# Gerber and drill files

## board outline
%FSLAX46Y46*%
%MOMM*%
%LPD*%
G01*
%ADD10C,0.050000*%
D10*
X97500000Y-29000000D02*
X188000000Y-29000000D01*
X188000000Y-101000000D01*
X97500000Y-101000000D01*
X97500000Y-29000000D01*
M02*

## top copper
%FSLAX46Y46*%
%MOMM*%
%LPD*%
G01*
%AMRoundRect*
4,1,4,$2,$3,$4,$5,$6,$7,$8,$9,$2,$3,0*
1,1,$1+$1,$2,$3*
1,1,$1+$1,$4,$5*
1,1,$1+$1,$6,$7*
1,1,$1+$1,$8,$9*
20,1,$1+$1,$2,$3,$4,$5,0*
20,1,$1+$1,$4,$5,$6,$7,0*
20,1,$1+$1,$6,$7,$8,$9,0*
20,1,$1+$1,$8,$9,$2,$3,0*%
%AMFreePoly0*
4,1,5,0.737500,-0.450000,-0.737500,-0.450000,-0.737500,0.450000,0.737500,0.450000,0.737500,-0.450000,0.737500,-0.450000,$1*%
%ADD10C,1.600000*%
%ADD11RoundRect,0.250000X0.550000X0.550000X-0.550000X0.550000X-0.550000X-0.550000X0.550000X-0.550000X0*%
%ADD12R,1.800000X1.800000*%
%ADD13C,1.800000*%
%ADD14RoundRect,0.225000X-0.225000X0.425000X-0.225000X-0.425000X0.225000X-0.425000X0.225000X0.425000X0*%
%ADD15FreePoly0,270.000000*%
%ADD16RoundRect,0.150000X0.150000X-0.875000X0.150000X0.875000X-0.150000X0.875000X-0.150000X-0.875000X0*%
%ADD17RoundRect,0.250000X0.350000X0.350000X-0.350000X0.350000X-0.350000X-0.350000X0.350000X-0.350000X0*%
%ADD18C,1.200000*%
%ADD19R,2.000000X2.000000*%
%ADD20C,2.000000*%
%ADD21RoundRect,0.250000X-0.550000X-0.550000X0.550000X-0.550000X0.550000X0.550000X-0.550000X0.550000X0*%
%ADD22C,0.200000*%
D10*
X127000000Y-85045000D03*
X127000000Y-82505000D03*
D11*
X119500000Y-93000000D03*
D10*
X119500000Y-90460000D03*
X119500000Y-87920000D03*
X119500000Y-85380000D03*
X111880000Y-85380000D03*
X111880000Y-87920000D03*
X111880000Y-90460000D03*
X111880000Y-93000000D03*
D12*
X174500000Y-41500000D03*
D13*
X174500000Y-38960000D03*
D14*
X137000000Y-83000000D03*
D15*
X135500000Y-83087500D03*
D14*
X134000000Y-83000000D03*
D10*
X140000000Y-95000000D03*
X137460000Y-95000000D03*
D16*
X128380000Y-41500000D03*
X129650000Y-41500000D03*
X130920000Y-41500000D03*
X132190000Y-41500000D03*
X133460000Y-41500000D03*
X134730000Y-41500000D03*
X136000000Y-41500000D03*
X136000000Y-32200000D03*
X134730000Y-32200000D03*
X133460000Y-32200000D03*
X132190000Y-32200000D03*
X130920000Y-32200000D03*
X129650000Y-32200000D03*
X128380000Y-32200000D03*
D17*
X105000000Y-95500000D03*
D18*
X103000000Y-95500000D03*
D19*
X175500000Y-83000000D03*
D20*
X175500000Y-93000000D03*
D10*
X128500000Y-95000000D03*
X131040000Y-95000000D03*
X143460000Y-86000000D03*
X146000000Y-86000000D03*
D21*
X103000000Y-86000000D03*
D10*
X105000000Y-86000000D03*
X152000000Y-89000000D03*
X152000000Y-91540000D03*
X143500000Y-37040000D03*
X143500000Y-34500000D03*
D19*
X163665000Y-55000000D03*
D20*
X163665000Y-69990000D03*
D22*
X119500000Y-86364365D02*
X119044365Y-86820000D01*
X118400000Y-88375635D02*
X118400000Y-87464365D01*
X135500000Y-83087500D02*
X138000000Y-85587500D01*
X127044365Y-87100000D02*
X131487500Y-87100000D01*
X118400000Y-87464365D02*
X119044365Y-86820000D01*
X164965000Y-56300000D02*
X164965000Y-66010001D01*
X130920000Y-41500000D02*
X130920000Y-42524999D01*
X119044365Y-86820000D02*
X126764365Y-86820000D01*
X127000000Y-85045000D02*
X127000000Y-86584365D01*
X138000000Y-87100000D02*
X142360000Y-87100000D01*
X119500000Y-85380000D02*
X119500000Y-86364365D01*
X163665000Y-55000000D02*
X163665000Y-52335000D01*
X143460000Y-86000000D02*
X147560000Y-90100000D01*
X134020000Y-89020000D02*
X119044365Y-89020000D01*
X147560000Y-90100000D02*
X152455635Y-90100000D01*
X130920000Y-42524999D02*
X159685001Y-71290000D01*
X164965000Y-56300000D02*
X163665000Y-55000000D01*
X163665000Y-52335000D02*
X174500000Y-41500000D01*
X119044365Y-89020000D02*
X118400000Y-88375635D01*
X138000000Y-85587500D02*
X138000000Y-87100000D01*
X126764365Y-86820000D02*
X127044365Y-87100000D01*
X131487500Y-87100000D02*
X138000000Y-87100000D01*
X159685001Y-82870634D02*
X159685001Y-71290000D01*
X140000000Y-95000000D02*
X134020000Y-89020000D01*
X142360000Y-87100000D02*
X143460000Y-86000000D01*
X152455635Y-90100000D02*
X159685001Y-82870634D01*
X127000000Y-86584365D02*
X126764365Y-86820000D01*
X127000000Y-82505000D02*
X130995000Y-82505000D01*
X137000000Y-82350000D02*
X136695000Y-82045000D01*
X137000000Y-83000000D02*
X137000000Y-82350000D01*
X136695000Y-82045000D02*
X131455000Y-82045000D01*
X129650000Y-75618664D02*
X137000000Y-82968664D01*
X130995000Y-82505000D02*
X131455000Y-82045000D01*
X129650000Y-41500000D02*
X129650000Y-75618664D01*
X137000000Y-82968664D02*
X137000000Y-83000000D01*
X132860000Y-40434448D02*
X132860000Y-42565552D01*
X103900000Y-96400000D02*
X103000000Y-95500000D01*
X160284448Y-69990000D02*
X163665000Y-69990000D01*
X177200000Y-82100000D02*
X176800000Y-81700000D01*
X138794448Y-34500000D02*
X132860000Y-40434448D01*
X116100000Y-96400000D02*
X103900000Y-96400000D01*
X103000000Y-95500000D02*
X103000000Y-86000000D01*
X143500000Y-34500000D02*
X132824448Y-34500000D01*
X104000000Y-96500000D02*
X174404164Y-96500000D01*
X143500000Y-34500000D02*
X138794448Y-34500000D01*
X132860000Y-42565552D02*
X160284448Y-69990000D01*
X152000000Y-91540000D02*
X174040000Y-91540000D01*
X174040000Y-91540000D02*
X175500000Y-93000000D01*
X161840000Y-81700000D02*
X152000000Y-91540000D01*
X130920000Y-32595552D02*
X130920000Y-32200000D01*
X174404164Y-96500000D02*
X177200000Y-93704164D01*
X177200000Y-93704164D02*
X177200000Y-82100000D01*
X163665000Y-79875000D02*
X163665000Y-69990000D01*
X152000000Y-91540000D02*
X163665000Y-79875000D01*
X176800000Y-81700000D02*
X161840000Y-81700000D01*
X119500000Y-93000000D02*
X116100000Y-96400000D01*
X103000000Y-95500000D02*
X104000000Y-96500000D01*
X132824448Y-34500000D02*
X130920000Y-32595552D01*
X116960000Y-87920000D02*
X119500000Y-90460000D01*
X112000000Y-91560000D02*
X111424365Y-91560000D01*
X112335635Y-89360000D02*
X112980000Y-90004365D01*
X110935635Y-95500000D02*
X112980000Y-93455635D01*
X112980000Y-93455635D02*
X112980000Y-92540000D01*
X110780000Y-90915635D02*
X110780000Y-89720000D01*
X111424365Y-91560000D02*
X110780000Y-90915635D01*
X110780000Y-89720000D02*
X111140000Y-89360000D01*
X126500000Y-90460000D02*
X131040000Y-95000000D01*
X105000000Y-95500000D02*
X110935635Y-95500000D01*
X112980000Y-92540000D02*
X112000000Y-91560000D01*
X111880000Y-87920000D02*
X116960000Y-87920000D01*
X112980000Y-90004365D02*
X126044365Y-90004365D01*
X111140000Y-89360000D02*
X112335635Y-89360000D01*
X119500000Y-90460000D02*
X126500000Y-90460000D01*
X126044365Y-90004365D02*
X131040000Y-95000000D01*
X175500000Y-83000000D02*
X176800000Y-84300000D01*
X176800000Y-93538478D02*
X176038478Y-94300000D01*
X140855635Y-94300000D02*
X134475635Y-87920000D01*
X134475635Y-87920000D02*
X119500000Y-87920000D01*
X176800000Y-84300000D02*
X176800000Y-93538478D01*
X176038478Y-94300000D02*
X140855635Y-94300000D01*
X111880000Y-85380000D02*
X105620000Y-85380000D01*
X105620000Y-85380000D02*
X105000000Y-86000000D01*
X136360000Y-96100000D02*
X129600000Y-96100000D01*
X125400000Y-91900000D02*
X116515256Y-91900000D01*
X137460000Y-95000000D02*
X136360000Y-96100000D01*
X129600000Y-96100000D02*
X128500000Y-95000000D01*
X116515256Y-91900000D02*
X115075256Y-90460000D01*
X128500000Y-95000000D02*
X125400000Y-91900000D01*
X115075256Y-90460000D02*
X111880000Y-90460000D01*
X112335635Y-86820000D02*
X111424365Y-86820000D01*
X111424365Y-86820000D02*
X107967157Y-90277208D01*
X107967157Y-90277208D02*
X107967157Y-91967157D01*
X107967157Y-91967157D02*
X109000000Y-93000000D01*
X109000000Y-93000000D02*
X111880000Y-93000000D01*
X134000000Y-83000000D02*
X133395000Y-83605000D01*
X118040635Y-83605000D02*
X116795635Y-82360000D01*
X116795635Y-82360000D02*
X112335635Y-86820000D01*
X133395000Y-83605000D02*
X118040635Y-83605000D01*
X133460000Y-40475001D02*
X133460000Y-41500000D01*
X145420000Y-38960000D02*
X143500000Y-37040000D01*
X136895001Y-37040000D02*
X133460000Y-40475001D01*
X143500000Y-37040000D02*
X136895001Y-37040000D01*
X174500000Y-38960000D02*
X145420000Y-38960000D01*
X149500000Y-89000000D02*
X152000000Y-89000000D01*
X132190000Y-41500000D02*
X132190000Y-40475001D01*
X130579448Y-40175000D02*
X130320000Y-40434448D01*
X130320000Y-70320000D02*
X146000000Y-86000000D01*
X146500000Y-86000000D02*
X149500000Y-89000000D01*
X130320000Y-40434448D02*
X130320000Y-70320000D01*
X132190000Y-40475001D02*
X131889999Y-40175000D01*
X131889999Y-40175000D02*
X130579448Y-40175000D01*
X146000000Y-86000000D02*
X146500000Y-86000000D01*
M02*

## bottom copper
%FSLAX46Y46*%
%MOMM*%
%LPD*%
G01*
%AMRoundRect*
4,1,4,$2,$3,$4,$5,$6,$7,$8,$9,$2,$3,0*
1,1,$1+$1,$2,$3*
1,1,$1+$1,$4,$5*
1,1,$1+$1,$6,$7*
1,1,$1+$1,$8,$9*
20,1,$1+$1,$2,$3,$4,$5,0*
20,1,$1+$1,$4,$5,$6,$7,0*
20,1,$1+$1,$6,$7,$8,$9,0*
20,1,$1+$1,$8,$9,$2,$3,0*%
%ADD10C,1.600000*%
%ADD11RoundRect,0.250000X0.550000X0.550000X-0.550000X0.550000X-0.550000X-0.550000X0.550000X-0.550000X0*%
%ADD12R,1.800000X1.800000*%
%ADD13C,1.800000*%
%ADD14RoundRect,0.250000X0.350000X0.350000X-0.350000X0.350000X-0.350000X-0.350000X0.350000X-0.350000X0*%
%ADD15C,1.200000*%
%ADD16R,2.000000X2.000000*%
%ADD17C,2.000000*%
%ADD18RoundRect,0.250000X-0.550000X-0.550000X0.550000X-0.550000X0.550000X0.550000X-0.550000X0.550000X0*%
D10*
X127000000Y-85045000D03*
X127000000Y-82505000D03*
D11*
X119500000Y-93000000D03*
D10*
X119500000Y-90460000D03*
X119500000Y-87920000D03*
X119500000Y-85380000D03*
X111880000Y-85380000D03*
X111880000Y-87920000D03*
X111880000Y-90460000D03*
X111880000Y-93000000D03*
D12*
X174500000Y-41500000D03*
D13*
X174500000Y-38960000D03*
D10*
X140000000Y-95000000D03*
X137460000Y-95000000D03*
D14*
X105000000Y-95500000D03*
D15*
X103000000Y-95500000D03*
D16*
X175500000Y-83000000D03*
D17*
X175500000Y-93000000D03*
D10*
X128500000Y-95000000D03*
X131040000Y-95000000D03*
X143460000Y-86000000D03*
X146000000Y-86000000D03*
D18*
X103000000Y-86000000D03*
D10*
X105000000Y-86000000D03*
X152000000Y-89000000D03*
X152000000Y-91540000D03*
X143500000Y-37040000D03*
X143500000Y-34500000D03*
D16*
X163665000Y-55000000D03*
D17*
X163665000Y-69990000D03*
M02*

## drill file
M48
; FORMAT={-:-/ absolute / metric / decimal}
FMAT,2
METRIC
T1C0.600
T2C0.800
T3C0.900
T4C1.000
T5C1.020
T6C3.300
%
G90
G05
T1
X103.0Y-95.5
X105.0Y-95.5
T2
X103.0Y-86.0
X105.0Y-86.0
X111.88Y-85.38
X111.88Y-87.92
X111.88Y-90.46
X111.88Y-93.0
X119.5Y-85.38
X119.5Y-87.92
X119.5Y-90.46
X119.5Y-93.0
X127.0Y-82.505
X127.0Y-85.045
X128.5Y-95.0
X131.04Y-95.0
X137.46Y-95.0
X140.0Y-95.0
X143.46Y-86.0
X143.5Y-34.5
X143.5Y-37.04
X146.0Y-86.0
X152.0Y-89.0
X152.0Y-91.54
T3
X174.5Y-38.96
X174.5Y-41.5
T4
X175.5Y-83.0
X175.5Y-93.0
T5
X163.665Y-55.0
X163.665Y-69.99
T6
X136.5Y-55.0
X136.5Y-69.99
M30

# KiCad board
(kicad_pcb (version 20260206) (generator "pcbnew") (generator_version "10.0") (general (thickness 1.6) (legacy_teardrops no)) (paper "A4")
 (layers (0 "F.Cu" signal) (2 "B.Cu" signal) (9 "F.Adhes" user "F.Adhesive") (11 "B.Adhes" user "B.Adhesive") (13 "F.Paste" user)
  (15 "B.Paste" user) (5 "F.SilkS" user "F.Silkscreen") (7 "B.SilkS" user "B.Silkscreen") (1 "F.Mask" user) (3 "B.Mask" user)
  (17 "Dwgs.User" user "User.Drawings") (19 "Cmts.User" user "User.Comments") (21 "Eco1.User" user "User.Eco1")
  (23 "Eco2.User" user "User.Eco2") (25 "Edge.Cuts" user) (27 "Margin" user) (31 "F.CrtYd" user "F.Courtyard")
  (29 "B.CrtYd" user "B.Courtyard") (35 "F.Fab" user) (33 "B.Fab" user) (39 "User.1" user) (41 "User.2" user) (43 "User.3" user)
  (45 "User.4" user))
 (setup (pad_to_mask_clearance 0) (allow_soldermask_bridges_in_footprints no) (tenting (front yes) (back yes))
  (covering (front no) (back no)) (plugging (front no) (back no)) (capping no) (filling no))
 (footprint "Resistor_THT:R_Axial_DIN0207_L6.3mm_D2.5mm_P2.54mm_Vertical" (layer "F.Cu") (at 127 85.045 90)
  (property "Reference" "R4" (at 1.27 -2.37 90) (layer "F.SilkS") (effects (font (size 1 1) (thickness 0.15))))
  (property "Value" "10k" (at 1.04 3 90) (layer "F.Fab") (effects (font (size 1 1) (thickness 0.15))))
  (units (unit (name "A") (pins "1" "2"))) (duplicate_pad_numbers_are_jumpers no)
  (pad "1" thru_hole circle (at 0 0 90) (size 1.6 1.6) (drill 0.8) (layers "*.Cu" "*.Mask") (remove_unused_layers no) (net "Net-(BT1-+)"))
  (pad "2" thru_hole circle (at 2.54 0 90) (size 1.6 1.6) (drill 0.8) (layers "*.Cu" "*.Mask") (remove_unused_layers no) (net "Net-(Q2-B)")))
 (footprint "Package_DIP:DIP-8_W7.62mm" (layer "F.Cu") (at 119.5 93 180)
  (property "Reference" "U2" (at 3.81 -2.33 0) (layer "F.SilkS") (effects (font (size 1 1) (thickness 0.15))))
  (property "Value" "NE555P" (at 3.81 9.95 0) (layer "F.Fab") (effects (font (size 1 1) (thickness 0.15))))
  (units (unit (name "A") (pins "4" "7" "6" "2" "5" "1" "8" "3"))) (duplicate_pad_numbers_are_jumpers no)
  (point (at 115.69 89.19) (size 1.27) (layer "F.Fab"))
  (pad "1" thru_hole roundrect (at 0 0 180) (size 1.6 1.6) (drill 0.8) (layers "*.Cu" "*.Mask") (remove_unused_layers no)
   (roundrect_rratio 0.15625) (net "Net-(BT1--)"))
  (pad "2" thru_hole circle (at 0 2.54 180) (size 1.6 1.6) (drill 0.8) (layers "*.Cu" "*.Mask") (remove_unused_layers no)
   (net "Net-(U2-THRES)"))
  (pad "3" thru_hole circle (at 0 5.08 180) (size 1.6 1.6) (drill 0.8) (layers "*.Cu" "*.Mask") (remove_unused_layers no)
   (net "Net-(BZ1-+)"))
  (pad "4" thru_hole circle (at 0 7.62 180) (size 1.6 1.6) (drill 0.8) (layers "*.Cu" "*.Mask") (remove_unused_layers no)
   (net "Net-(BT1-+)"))
  (pad "5" thru_hole circle (at 7.62 7.62 180) (size 1.6 1.6) (drill 0.8) (layers "*.Cu" "*.Mask") (remove_unused_layers no)
   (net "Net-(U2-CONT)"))
  (pad "6" thru_hole circle (at 7.62 5.08 180) (size 1.6 1.6) (drill 0.8) (layers "*.Cu" "*.Mask") (remove_unused_layers no)
   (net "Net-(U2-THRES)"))
  (pad "7" thru_hole circle (at 7.62 2.54 180) (size 1.6 1.6) (drill 0.8) (layers "*.Cu" "*.Mask") (remove_unused_layers no)
   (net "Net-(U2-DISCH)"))
  (pad "8" thru_hole circle (at 7.62 0 180) (size 1.6 1.6) (drill 0.8) (layers "*.Cu" "*.Mask") (remove_unused_layers no) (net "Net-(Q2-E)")))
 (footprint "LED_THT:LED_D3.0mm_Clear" (layer "F.Cu") (at 174.5 41.5 90)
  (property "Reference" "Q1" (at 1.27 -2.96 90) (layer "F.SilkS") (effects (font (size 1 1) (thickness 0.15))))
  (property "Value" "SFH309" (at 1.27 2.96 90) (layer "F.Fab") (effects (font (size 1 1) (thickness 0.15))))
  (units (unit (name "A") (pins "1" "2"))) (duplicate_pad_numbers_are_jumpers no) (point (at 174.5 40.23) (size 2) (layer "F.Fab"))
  (pad "1" thru_hole rect (at 0 0 90) (size 1.8 1.8) (drill 0.9) (layers "*.Cu" "*.Mask") (remove_unused_layers no) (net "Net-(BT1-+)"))
  (pad "2" thru_hole circle (at 2.54 0 90) (size 1.8 1.8) (drill 0.9) (layers "*.Cu" "*.Mask") (remove_unused_layers no) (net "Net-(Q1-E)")))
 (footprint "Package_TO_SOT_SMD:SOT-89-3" (layer "F.Cu") (at 135.5 84.95 -90)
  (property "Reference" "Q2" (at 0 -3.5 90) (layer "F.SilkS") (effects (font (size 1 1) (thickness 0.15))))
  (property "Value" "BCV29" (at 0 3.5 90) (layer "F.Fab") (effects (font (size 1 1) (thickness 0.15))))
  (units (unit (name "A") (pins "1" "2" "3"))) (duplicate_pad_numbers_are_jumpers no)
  (pad "1" smd roundrect (at -1.95 -1.5 270) (size 1.3 0.9) (layers "F.Cu" "F.Mask" "F.Paste") (roundrect_rratio 0.25) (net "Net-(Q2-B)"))
  (pad "2" smd custom (at -1.8625 0 270) (size 1.475 0.9) (layers "F.Cu" "F.Mask" "F.Paste") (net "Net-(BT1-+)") (zone_connect 2)
   (thermal_bridge_angle 45) (options (clearance outline) (anchor rect)) (primitives))
  (pad "3" smd roundrect (at -1.95 1.5 270) (size 1.3 0.9) (layers "F.Cu" "F.Mask" "F.Paste") (roundrect_rratio 0.25) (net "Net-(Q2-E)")))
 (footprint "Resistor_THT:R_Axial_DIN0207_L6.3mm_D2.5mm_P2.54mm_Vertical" (layer "F.Cu") (at 140 95 180)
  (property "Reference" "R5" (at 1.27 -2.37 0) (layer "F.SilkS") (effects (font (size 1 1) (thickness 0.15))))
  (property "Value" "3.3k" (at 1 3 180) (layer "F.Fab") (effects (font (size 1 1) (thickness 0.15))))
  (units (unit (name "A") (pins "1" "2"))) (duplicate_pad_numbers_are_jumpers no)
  (pad "1" thru_hole circle (at 0 0 180) (size 1.6 1.6) (drill 0.8) (layers "*.Cu" "*.Mask") (remove_unused_layers no) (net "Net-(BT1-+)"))
  (pad "2" thru_hole circle (at 2.54 0 180) (size 1.6 1.6) (drill 0.8) (layers "*.Cu" "*.Mask") (remove_unused_layers no)
   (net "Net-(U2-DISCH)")))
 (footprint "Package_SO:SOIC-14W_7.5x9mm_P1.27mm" (layer "F.Cu") (at 132.19 36.85 90)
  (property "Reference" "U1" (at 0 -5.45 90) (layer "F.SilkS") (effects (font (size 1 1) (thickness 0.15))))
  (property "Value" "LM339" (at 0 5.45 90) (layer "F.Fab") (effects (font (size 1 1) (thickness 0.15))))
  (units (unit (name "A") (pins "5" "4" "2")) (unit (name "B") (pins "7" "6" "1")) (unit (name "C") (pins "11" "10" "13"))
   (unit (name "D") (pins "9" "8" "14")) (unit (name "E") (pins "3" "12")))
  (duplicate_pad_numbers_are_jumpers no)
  (pad "1" smd roundrect (at -4.65 -3.81 90) (size 2.05 0.6) (layers "F.Cu" "F.Mask" "F.Paste") (roundrect_rratio 0.25))
  (pad "2" smd roundrect (at -4.65 -2.54 90) (size 2.05 0.6) (layers "F.Cu" "F.Mask" "F.Paste") (roundrect_rratio 0.25) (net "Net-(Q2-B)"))
  (pad "3" smd roundrect (at -4.65 -1.27 90) (size 2.05 0.6) (layers "F.Cu" "F.Mask" "F.Paste") (roundrect_rratio 0.25) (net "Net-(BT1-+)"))
  (pad "4" smd roundrect (at -4.65 0 90) (size 2.05 0.6) (layers "F.Cu" "F.Mask" "F.Paste") (roundrect_rratio 0.25) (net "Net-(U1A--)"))
  (pad "5" smd roundrect (at -4.65 1.27 90) (size 2.05 0.6) (layers "F.Cu" "F.Mask" "F.Paste") (roundrect_rratio 0.25) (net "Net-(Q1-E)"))
  (pad "6" smd roundrect (at -4.65 2.54 90) (size 2.05 0.6) (layers "F.Cu" "F.Mask" "F.Paste") (roundrect_rratio 0.25))
  (pad "7" smd roundrect (at -4.65 3.81 90) (size 2.05 0.6) (layers "F.Cu" "F.Mask" "F.Paste") (roundrect_rratio 0.25))
  (pad "8" smd roundrect (at 4.65 3.81 90) (size 2.05 0.6) (layers "F.Cu" "F.Mask" "F.Paste") (roundrect_rratio 0.25))
  (pad "9" smd roundrect (at 4.65 2.54 90) (size 2.05 0.6) (layers "F.Cu" "F.Mask" "F.Paste") (roundrect_rratio 0.25))
  (pad "10" smd roundrect (at 4.65 1.27 90) (size 2.05 0.6) (layers "F.Cu" "F.Mask" "F.Paste") (roundrect_rratio 0.25))
  (pad "11" smd roundrect (at 4.65 0 90) (size 2.05 0.6) (layers "F.Cu" "F.Mask" "F.Paste") (roundrect_rratio 0.25))
  (pad "12" smd roundrect (at 4.65 -1.27 90) (size 2.05 0.6) (layers "F.Cu" "F.Mask" "F.Paste") (roundrect_rratio 0.25) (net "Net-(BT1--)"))
  (pad "13" smd roundrect (at 4.65 -2.54 90) (size 2.05 0.6) (layers "F.Cu" "F.Mask" "F.Paste") (roundrect_rratio 0.25))
  (pad "14" smd roundrect (at 4.65 -3.81 90) (size 2.05 0.6) (layers "F.Cu" "F.Mask" "F.Paste") (roundrect_rratio 0.25)))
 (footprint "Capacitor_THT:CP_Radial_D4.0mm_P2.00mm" (layer "F.Cu") (at 105 95.5 180)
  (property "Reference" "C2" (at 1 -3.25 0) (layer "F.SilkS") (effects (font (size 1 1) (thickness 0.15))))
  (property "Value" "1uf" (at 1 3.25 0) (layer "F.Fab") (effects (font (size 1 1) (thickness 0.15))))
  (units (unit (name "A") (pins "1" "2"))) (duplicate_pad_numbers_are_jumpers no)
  (pad "1" thru_hole roundrect (at 0 0 180) (size 1.2 1.2) (drill 0.6) (layers "*.Cu" "*.Mask") (remove_unused_layers no)
   (roundrect_rratio 0.208333) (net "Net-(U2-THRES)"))
  (pad "2" thru_hole circle (at 2 0 180) (size 1.2 1.2) (drill 0.6) (layers "*.Cu" "*.Mask") (remove_unused_layers no) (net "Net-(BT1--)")))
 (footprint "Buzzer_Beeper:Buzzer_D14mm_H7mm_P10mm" (layer "F.Cu") (at 175.5 83 -90)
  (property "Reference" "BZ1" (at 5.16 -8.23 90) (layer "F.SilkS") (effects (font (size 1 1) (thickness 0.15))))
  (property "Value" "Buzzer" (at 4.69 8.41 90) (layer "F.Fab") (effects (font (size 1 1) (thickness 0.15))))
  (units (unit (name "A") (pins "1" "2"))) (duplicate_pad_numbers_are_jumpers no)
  (pad "1" thru_hole rect (at 0 0 270) (size 2 2) (drill 1) (layers "*.Cu" "*.Mask") (remove_unused_layers no) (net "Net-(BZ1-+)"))
  (pad "2" thru_hole circle (at 10 0 270) (size 2 2) (drill 1) (layers "*.Cu" "*.Mask") (remove_unused_layers no) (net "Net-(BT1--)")))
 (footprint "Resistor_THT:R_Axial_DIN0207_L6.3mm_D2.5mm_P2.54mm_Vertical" (layer "F.Cu") (at 128.5 95)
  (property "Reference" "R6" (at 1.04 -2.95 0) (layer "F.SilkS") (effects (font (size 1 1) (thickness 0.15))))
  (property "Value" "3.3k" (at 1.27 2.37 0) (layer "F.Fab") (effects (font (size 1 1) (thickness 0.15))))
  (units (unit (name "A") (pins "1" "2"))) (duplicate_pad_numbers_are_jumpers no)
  (pad "1" thru_hole circle (at 0 0) (size 1.6 1.6) (drill 0.8) (layers "*.Cu" "*.Mask") (remove_unused_layers no) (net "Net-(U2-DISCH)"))
  (pad "2" thru_hole circle (at 2.54 0) (size 1.6 1.6) (drill 0.8) (layers "*.Cu" "*.Mask") (remove_unused_layers no) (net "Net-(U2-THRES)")))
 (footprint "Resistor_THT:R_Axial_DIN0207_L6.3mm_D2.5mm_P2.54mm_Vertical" (layer "F.Cu") (at 143.46 86)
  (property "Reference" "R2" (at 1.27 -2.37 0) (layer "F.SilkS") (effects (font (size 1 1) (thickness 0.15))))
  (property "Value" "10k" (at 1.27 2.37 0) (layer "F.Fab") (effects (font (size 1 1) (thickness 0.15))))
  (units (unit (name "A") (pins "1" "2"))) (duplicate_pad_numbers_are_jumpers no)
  (pad "1" thru_hole circle (at 0 0) (size 1.6 1.6) (drill 0.8) (layers "*.Cu" "*.Mask") (remove_unused_layers no) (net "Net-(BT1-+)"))
  (pad "2" thru_hole circle (at 2.54 0) (size 1.6 1.6) (drill 0.8) (layers "*.Cu" "*.Mask") (remove_unused_layers no) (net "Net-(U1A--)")))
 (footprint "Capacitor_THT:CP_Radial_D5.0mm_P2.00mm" (layer "F.Cu") (at 103 86)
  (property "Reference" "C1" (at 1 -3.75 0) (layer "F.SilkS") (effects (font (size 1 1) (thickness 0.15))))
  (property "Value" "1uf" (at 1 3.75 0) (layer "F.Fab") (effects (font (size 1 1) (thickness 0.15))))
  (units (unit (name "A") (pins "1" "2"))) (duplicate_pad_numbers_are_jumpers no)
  (pad "1" thru_hole roundrect (at 0 0) (size 1.6 1.6) (drill 0.8) (layers "*.Cu" "*.Mask") (remove_unused_layers no)
   (roundrect_rratio 0.15625) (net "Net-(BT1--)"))
  (pad "2" thru_hole circle (at 2 0) (size 1.6 1.6) (drill 0.8) (layers "*.Cu" "*.Mask") (remove_unused_layers no) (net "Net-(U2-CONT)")))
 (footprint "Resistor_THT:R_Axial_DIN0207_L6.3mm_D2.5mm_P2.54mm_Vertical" (layer "F.Cu") (at 152 89 -90)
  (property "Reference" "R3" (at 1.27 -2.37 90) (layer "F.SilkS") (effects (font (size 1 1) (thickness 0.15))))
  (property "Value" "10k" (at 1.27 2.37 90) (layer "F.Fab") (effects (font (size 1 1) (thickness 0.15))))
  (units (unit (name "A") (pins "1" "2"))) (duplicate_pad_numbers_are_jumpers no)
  (pad "1" thru_hole circle (at 0 0 270) (size 1.6 1.6) (drill 0.8) (layers "*.Cu" "*.Mask") (remove_unused_layers no) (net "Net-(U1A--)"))
  (pad "2" thru_hole circle (at 2.54 0 270) (size 1.6 1.6) (drill 0.8) (layers "*.Cu" "*.Mask") (remove_unused_layers no)
   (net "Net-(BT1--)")))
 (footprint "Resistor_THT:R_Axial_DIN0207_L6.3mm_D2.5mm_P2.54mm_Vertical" (layer "F.Cu") (at 143.5 37.04 90)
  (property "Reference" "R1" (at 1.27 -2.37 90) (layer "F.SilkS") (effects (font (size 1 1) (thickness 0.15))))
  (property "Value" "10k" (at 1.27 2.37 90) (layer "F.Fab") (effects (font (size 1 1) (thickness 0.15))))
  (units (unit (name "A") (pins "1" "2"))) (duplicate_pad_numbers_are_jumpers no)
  (pad "1" thru_hole circle (at 0 0 90) (size 1.6 1.6) (drill 0.8) (layers "*.Cu" "*.Mask") (remove_unused_layers no) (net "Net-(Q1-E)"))
  (pad "2" thru_hole circle (at 2.54 0 90) (size 1.6 1.6) (drill 0.8) (layers "*.Cu" "*.Mask") (remove_unused_layers no) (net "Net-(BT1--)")))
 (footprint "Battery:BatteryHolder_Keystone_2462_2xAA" (layer "B.Cu") (at 163.665 55 180)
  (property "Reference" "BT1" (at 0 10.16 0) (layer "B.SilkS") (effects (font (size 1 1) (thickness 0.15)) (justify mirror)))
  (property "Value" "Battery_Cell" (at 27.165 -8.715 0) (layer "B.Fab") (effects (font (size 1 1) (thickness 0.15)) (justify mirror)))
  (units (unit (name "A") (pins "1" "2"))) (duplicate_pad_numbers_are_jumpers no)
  (pad "" np_thru_hole circle (at 27.165 -14.99 180) (size 3.3 3.3) (drill 3.3) (layers "*.Cu" "*.Mask"))
  (pad "" np_thru_hole circle (at 27.165 0 180) (size 3.3 3.3) (drill 3.3) (layers "*.Cu" "*.Mask"))
  (pad "1" thru_hole rect (at 0 0 180) (size 2 2) (drill 1.02) (layers "*.Cu" "*.Mask") (remove_unused_layers no) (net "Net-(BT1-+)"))
  (pad "2" thru_hole circle (at 0 -14.99 180) (size 2 2) (drill 1.02) (layers "*.Cu" "*.Mask") (remove_unused_layers no) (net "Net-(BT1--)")))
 (gr_rect (start 97.5 29) (end 188 101) (stroke (width 0.05) (type default)) (fill no) (layer "Edge.Cuts"))
 (segment (start 119.5 86.364365) (end 119.044365 86.82) (width 0.2) (layer "F.Cu") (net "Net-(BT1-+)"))
 (segment (start 118.4 88.375635) (end 118.4 87.464365) (width 0.2) (layer "F.Cu") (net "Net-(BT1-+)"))
 (segment (start 135.5 83.0875) (end 138 85.5875) (width 0.2) (layer "F.Cu") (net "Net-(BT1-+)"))
 (segment (start 127.044365 87.1) (end 131.4875 87.1) (width 0.2) (layer "F.Cu") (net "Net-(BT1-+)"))
 (segment (start 118.4 87.464365) (end 119.044365 86.82) (width 0.2) (layer "F.Cu") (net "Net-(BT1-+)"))
 (segment (start 164.965 56.3) (end 164.965 66.010001) (width 0.2) (layer "F.Cu") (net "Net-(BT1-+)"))
 (segment (start 130.92 41.5) (end 130.92 42.524999) (width 0.2) (layer "F.Cu") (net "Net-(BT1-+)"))
 (segment (start 119.044365 86.82) (end 126.764365 86.82) (width 0.2) (layer "F.Cu") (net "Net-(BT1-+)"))
 (segment (start 127 85.045) (end 127 86.584365) (width 0.2) (layer "F.Cu") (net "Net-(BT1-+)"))
 (segment (start 138 87.1) (end 142.36 87.1) (width 0.2) (layer "F.Cu") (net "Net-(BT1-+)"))
 (segment (start 119.5 85.38) (end 119.5 86.364365) (width 0.2) (layer "F.Cu") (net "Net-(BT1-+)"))
 (segment (start 163.665 55) (end 163.665 52.335) (width 0.2) (layer "F.Cu") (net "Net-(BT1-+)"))
 (segment (start 143.46 86) (end 147.56 90.1) (width 0.2) (layer "F.Cu") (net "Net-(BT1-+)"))
 (segment (start 134.02 89.02) (end 119.044365 89.02) (width 0.2) (layer "F.Cu") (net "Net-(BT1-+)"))
 (segment (start 147.56 90.1) (end 152.455635 90.1) (width 0.2) (layer "F.Cu") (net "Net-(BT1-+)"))
 (segment (start 130.92 42.524999) (end 159.685001 71.29) (width 0.2) (layer "F.Cu") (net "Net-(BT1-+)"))
 (segment (start 164.965 56.3) (end 163.665 55) (width 0.2) (layer "F.Cu") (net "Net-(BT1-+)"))
 (segment (start 163.665 52.335) (end 174.5 41.5) (width 0.2) (layer "F.Cu") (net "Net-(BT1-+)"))
 (segment (start 119.044365 89.02) (end 118.4 88.375635) (width 0.2) (layer "F.Cu") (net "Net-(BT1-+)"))
 (segment (start 138 85.5875) (end 138 87.1) (width 0.2) (layer "F.Cu") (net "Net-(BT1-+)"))
 (segment (start 126.764365 86.82) (end 127.044365 87.1) (width 0.2) (layer "F.Cu") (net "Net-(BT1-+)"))
 (segment (start 131.4875 87.1) (end 138 87.1) (width 0.2) (layer "F.Cu") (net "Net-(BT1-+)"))
 (segment (start 159.685001 82.870634) (end 159.685001 71.29) (width 0.2) (layer "F.Cu") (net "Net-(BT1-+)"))
 (segment (start 140 95) (end 134.02 89.02) (width 0.2) (layer "F.Cu") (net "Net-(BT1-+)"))
 (segment (start 142.36 87.1) (end 143.46 86) (width 0.2) (layer "F.Cu") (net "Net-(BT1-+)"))
 (segment (start 152.455635 90.1) (end 159.685001 82.870634) (width 0.2) (layer "F.Cu") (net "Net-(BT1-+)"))
 (segment (start 127 86.584365) (end 126.764365 86.82) (width 0.2) (layer "F.Cu") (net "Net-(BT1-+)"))
 (segment (start 127 82.505) (end 130.995 82.505) (width 0.2) (layer "F.Cu") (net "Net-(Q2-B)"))
 (segment (start 137 82.35) (end 136.695 82.045) (width 0.2) (layer "F.Cu") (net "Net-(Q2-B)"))
 (segment (start 137 83) (end 137 82.35) (width 0.2) (layer "F.Cu") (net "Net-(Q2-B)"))
 (segment (start 136.695 82.045) (end 131.455 82.045) (width 0.2) (layer "F.Cu") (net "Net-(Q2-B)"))
 (segment (start 129.65 75.618664) (end 137 82.968664) (width 0.2) (layer "F.Cu") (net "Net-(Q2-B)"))
 (segment (start 130.995 82.505) (end 131.455 82.045) (width 0.2) (layer "F.Cu") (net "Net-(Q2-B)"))
 (segment (start 129.65 41.5) (end 129.65 75.618664) (width 0.2) (layer "F.Cu") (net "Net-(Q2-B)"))
 (segment (start 137 82.968664) (end 137 83) (width 0.2) (layer "F.Cu") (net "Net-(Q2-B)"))
 (segment (start 132.86 40.434448) (end 132.86 42.565552) (width 0.2) (layer "F.Cu") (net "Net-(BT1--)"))
 (segment (start 103.9 96.4) (end 103 95.5) (width 0.2) (layer "F.Cu") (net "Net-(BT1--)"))
 (segment (start 160.284448 69.99) (end 163.665 69.99) (width 0.2) (layer "F.Cu") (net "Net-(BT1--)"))
 (segment (start 177.2 82.1) (end 176.8 81.7) (width 0.2) (layer "F.Cu") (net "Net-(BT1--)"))
 (segment (start 138.794448 34.5) (end 132.86 40.434448) (width 0.2) (layer "F.Cu") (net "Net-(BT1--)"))
 (segment (start 116.1 96.4) (end 103.9 96.4) (width 0.2) (layer "F.Cu") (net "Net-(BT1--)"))
 (segment (start 103 95.5) (end 103 86) (width 0.2) (layer "F.Cu") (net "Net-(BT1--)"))
 (segment (start 143.5 34.5) (end 132.824448 34.5) (width 0.2) (layer "F.Cu") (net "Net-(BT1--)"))
 (segment (start 104 96.5) (end 174.404164 96.5) (width 0.2) (layer "F.Cu") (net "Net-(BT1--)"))
 (segment (start 143.5 34.5) (end 138.794448 34.5) (width 0.2) (layer "F.Cu") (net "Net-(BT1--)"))
 (segment (start 132.86 42.565552) (end 160.284448 69.99) (width 0.2) (layer "F.Cu") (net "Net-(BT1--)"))
 (segment (start 152 91.54) (end 174.04 91.54) (width 0.2) (layer "F.Cu") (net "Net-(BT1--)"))
 (segment (start 174.04 91.54) (end 175.5 93) (width 0.2) (layer "F.Cu") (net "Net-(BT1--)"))
 (segment (start 161.84 81.7) (end 152 91.54) (width 0.2) (layer "F.Cu") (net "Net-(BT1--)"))
 (segment (start 130.92 32.595552) (end 130.92 32.2) (width 0.2) (layer "F.Cu") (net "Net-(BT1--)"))
 (segment (start 174.404164 96.5) (end 177.2 93.704164) (width 0.2) (layer "F.Cu") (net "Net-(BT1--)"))
 (segment (start 177.2 93.704164) (end 177.2 82.1) (width 0.2) (layer "F.Cu") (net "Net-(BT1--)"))
 (segment (start 163.665 79.875) (end 163.665 69.99) (width 0.2) (layer "F.Cu") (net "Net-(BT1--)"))
 (segment (start 152 91.54) (end 163.665 79.875) (width 0.2) (layer "F.Cu") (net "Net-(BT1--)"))
 (segment (start 176.8 81.7) (end 161.84 81.7) (width 0.2) (layer "F.Cu") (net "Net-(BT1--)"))
 (segment (start 119.5 93) (end 116.1 96.4) (width 0.2) (layer "F.Cu") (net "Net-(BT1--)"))
 (segment (start 103 95.5) (end 104 96.5) (width 0.2) (layer "F.Cu") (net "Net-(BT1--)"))
 (segment (start 132.824448 34.5) (end 130.92 32.595552) (width 0.2) (layer "F.Cu") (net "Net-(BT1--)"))
 (segment (start 116.96 87.92) (end 119.5 90.46) (width 0.2) (layer "F.Cu") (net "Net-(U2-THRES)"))
 (segment (start 112 91.56) (end 111.424365 91.56) (width 0.2) (layer "F.Cu") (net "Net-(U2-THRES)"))
 (segment (start 112.335635 89.36) (end 112.98 90.004365) (width 0.2) (layer "F.Cu") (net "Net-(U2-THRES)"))
 (segment (start 110.935635 95.5) (end 112.98 93.455635) (width 0.2) (layer "F.Cu") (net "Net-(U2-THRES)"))
 (segment (start 112.98 93.455635) (end 112.98 92.54) (width 0.2) (layer "F.Cu") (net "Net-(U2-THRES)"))
 (segment (start 110.78 90.915635) (end 110.78 89.72) (width 0.2) (layer "F.Cu") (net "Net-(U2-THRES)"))
 (segment (start 111.424365 91.56) (end 110.78 90.915635) (width 0.2) (layer "F.Cu") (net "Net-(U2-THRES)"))
 (segment (start 110.78 89.72) (end 111.14 89.36) (width 0.2) (layer "F.Cu") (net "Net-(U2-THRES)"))
 (segment (start 126.5 90.46) (end 131.04 95) (width 0.2) (layer "F.Cu") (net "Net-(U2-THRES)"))
 (segment (start 105 95.5) (end 110.935635 95.5) (width 0.2) (layer "F.Cu") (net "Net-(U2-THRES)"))
 (segment (start 112.98 92.54) (end 112 91.56) (width 0.2) (layer "F.Cu") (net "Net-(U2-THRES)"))
 (segment (start 111.88 87.92) (end 116.96 87.92) (width 0.2) (layer "F.Cu") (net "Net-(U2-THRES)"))
 (segment (start 112.98 90.004365) (end 126.044365 90.004365) (width 0.2) (layer "F.Cu") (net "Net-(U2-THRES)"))
 (segment (start 111.14 89.36) (end 112.335635 89.36) (width 0.2) (layer "F.Cu") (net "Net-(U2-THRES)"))
 (segment (start 119.5 90.46) (end 126.5 90.46) (width 0.2) (layer "F.Cu") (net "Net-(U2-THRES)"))
 (segment (start 126.044365 90.004365) (end 131.04 95) (width 0.2) (layer "F.Cu") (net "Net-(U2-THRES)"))
 (segment (start 175.5 83) (end 176.8 84.3) (width 0.2) (layer "F.Cu") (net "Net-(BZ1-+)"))
 (segment (start 176.8 93.538478) (end 176.038478 94.3) (width 0.2) (layer "F.Cu") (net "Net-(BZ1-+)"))
 (segment (start 140.855635 94.3) (end 134.475635 87.92) (width 0.2) (layer "F.Cu") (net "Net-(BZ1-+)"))
 (segment (start 134.475635 87.92) (end 119.5 87.92) (width 0.2) (layer "F.Cu") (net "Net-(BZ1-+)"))
 (segment (start 176.8 84.3) (end 176.8 93.538478) (width 0.2) (layer "F.Cu") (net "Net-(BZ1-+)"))
 (segment (start 176.038478 94.3) (end 140.855635 94.3) (width 0.2) (layer "F.Cu") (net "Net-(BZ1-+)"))
 (segment (start 111.88 85.38) (end 105.62 85.38) (width 0.2) (layer "F.Cu") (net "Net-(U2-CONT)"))
 (segment (start 105.62 85.38) (end 105 86) (width 0.2) (layer "F.Cu") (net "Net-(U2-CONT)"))
 (segment (start 136.36 96.1) (end 129.6 96.1) (width 0.2) (layer "F.Cu") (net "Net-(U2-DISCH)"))
 (segment (start 125.4 91.9) (end 116.515256 91.9) (width 0.2) (layer "F.Cu") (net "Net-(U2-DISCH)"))
 (segment (start 137.46 95) (end 136.36 96.1) (width 0.2) (layer "F.Cu") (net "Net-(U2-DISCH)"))
 (segment (start 129.6 96.1) (end 128.5 95) (width 0.2) (layer "F.Cu") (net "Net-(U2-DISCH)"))
 (segment (start 116.515256 91.9) (end 115.075256 90.46) (width 0.2) (layer "F.Cu") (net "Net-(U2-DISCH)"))
 (segment (start 128.5 95) (end 125.4 91.9) (width 0.2) (layer "F.Cu") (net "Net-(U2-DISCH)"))
 (segment (start 115.075256 90.46) (end 111.88 90.46) (width 0.2) (layer "F.Cu") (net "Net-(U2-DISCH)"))
 (segment (start 112.335635 86.82) (end 111.424365 86.82) (width 0.2) (layer "F.Cu") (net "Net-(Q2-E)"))
 (segment (start 111.424365 86.82) (end 107.967157 90.277208) (width 0.2) (layer "F.Cu") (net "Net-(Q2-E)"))
 (segment (start 107.967157 90.277208) (end 107.967157 91.967157) (width 0.2) (layer "F.Cu") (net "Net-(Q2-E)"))
 (segment (start 107.967157 91.967157) (end 109 93) (width 0.2) (layer "F.Cu") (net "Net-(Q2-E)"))
 (segment (start 109 93) (end 111.88 93) (width 0.2) (layer "F.Cu") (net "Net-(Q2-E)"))
 (segment (start 134 83) (end 133.395 83.605) (width 0.2) (layer "F.Cu") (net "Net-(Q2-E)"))
 (segment (start 118.040635 83.605) (end 116.795635 82.36) (width 0.2) (layer "F.Cu") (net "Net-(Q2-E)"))
 (segment (start 116.795635 82.36) (end 112.335635 86.82) (width 0.2) (layer "F.Cu") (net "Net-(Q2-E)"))
 (segment (start 133.395 83.605) (end 118.040635 83.605) (width 0.2) (layer "F.Cu") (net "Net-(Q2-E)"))
 (segment (start 133.46 40.475001) (end 133.46 41.5) (width 0.2) (layer "F.Cu") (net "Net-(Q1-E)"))
 (segment (start 145.42 38.96) (end 143.5 37.04) (width 0.2) (layer "F.Cu") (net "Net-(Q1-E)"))
 (segment (start 136.895001 37.04) (end 133.46 40.475001) (width 0.2) (layer "F.Cu") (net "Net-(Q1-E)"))
 (segment (start 143.5 37.04) (end 136.895001 37.04) (width 0.2) (layer "F.Cu") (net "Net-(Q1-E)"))
 (segment (start 174.5 38.96) (end 145.42 38.96) (width 0.2) (layer "F.Cu") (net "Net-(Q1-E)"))
 (segment (start 149.5 89) (end 152 89) (width 0.2) (layer "F.Cu") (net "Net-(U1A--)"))
 (segment (start 132.19 41.5) (end 132.19 40.475001) (width 0.2) (layer "F.Cu") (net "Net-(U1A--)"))
 (segment (start 130.579448 40.175) (end 130.32 40.434448) (width 0.2) (layer "F.Cu") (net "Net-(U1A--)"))
 (segment (start 130.32 70.32) (end 146 86) (width 0.2) (layer "F.Cu") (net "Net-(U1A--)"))
 (segment (start 146.5 86) (end 149.5 89) (width 0.2) (layer "F.Cu") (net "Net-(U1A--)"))
 (segment (start 130.32 40.434448) (end 130.32 70.32) (width 0.2) (layer "F.Cu") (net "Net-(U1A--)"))
 (segment (start 132.19 40.475001) (end 131.889999 40.175) (width 0.2) (layer "F.Cu") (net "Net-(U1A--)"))
 (segment (start 131.889999 40.175) (end 130.579448 40.175) (width 0.2) (layer "F.Cu") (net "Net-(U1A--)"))
 (segment (start 146 86) (end 146.5 86) (width 0.2) (layer "F.Cu") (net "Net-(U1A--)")))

